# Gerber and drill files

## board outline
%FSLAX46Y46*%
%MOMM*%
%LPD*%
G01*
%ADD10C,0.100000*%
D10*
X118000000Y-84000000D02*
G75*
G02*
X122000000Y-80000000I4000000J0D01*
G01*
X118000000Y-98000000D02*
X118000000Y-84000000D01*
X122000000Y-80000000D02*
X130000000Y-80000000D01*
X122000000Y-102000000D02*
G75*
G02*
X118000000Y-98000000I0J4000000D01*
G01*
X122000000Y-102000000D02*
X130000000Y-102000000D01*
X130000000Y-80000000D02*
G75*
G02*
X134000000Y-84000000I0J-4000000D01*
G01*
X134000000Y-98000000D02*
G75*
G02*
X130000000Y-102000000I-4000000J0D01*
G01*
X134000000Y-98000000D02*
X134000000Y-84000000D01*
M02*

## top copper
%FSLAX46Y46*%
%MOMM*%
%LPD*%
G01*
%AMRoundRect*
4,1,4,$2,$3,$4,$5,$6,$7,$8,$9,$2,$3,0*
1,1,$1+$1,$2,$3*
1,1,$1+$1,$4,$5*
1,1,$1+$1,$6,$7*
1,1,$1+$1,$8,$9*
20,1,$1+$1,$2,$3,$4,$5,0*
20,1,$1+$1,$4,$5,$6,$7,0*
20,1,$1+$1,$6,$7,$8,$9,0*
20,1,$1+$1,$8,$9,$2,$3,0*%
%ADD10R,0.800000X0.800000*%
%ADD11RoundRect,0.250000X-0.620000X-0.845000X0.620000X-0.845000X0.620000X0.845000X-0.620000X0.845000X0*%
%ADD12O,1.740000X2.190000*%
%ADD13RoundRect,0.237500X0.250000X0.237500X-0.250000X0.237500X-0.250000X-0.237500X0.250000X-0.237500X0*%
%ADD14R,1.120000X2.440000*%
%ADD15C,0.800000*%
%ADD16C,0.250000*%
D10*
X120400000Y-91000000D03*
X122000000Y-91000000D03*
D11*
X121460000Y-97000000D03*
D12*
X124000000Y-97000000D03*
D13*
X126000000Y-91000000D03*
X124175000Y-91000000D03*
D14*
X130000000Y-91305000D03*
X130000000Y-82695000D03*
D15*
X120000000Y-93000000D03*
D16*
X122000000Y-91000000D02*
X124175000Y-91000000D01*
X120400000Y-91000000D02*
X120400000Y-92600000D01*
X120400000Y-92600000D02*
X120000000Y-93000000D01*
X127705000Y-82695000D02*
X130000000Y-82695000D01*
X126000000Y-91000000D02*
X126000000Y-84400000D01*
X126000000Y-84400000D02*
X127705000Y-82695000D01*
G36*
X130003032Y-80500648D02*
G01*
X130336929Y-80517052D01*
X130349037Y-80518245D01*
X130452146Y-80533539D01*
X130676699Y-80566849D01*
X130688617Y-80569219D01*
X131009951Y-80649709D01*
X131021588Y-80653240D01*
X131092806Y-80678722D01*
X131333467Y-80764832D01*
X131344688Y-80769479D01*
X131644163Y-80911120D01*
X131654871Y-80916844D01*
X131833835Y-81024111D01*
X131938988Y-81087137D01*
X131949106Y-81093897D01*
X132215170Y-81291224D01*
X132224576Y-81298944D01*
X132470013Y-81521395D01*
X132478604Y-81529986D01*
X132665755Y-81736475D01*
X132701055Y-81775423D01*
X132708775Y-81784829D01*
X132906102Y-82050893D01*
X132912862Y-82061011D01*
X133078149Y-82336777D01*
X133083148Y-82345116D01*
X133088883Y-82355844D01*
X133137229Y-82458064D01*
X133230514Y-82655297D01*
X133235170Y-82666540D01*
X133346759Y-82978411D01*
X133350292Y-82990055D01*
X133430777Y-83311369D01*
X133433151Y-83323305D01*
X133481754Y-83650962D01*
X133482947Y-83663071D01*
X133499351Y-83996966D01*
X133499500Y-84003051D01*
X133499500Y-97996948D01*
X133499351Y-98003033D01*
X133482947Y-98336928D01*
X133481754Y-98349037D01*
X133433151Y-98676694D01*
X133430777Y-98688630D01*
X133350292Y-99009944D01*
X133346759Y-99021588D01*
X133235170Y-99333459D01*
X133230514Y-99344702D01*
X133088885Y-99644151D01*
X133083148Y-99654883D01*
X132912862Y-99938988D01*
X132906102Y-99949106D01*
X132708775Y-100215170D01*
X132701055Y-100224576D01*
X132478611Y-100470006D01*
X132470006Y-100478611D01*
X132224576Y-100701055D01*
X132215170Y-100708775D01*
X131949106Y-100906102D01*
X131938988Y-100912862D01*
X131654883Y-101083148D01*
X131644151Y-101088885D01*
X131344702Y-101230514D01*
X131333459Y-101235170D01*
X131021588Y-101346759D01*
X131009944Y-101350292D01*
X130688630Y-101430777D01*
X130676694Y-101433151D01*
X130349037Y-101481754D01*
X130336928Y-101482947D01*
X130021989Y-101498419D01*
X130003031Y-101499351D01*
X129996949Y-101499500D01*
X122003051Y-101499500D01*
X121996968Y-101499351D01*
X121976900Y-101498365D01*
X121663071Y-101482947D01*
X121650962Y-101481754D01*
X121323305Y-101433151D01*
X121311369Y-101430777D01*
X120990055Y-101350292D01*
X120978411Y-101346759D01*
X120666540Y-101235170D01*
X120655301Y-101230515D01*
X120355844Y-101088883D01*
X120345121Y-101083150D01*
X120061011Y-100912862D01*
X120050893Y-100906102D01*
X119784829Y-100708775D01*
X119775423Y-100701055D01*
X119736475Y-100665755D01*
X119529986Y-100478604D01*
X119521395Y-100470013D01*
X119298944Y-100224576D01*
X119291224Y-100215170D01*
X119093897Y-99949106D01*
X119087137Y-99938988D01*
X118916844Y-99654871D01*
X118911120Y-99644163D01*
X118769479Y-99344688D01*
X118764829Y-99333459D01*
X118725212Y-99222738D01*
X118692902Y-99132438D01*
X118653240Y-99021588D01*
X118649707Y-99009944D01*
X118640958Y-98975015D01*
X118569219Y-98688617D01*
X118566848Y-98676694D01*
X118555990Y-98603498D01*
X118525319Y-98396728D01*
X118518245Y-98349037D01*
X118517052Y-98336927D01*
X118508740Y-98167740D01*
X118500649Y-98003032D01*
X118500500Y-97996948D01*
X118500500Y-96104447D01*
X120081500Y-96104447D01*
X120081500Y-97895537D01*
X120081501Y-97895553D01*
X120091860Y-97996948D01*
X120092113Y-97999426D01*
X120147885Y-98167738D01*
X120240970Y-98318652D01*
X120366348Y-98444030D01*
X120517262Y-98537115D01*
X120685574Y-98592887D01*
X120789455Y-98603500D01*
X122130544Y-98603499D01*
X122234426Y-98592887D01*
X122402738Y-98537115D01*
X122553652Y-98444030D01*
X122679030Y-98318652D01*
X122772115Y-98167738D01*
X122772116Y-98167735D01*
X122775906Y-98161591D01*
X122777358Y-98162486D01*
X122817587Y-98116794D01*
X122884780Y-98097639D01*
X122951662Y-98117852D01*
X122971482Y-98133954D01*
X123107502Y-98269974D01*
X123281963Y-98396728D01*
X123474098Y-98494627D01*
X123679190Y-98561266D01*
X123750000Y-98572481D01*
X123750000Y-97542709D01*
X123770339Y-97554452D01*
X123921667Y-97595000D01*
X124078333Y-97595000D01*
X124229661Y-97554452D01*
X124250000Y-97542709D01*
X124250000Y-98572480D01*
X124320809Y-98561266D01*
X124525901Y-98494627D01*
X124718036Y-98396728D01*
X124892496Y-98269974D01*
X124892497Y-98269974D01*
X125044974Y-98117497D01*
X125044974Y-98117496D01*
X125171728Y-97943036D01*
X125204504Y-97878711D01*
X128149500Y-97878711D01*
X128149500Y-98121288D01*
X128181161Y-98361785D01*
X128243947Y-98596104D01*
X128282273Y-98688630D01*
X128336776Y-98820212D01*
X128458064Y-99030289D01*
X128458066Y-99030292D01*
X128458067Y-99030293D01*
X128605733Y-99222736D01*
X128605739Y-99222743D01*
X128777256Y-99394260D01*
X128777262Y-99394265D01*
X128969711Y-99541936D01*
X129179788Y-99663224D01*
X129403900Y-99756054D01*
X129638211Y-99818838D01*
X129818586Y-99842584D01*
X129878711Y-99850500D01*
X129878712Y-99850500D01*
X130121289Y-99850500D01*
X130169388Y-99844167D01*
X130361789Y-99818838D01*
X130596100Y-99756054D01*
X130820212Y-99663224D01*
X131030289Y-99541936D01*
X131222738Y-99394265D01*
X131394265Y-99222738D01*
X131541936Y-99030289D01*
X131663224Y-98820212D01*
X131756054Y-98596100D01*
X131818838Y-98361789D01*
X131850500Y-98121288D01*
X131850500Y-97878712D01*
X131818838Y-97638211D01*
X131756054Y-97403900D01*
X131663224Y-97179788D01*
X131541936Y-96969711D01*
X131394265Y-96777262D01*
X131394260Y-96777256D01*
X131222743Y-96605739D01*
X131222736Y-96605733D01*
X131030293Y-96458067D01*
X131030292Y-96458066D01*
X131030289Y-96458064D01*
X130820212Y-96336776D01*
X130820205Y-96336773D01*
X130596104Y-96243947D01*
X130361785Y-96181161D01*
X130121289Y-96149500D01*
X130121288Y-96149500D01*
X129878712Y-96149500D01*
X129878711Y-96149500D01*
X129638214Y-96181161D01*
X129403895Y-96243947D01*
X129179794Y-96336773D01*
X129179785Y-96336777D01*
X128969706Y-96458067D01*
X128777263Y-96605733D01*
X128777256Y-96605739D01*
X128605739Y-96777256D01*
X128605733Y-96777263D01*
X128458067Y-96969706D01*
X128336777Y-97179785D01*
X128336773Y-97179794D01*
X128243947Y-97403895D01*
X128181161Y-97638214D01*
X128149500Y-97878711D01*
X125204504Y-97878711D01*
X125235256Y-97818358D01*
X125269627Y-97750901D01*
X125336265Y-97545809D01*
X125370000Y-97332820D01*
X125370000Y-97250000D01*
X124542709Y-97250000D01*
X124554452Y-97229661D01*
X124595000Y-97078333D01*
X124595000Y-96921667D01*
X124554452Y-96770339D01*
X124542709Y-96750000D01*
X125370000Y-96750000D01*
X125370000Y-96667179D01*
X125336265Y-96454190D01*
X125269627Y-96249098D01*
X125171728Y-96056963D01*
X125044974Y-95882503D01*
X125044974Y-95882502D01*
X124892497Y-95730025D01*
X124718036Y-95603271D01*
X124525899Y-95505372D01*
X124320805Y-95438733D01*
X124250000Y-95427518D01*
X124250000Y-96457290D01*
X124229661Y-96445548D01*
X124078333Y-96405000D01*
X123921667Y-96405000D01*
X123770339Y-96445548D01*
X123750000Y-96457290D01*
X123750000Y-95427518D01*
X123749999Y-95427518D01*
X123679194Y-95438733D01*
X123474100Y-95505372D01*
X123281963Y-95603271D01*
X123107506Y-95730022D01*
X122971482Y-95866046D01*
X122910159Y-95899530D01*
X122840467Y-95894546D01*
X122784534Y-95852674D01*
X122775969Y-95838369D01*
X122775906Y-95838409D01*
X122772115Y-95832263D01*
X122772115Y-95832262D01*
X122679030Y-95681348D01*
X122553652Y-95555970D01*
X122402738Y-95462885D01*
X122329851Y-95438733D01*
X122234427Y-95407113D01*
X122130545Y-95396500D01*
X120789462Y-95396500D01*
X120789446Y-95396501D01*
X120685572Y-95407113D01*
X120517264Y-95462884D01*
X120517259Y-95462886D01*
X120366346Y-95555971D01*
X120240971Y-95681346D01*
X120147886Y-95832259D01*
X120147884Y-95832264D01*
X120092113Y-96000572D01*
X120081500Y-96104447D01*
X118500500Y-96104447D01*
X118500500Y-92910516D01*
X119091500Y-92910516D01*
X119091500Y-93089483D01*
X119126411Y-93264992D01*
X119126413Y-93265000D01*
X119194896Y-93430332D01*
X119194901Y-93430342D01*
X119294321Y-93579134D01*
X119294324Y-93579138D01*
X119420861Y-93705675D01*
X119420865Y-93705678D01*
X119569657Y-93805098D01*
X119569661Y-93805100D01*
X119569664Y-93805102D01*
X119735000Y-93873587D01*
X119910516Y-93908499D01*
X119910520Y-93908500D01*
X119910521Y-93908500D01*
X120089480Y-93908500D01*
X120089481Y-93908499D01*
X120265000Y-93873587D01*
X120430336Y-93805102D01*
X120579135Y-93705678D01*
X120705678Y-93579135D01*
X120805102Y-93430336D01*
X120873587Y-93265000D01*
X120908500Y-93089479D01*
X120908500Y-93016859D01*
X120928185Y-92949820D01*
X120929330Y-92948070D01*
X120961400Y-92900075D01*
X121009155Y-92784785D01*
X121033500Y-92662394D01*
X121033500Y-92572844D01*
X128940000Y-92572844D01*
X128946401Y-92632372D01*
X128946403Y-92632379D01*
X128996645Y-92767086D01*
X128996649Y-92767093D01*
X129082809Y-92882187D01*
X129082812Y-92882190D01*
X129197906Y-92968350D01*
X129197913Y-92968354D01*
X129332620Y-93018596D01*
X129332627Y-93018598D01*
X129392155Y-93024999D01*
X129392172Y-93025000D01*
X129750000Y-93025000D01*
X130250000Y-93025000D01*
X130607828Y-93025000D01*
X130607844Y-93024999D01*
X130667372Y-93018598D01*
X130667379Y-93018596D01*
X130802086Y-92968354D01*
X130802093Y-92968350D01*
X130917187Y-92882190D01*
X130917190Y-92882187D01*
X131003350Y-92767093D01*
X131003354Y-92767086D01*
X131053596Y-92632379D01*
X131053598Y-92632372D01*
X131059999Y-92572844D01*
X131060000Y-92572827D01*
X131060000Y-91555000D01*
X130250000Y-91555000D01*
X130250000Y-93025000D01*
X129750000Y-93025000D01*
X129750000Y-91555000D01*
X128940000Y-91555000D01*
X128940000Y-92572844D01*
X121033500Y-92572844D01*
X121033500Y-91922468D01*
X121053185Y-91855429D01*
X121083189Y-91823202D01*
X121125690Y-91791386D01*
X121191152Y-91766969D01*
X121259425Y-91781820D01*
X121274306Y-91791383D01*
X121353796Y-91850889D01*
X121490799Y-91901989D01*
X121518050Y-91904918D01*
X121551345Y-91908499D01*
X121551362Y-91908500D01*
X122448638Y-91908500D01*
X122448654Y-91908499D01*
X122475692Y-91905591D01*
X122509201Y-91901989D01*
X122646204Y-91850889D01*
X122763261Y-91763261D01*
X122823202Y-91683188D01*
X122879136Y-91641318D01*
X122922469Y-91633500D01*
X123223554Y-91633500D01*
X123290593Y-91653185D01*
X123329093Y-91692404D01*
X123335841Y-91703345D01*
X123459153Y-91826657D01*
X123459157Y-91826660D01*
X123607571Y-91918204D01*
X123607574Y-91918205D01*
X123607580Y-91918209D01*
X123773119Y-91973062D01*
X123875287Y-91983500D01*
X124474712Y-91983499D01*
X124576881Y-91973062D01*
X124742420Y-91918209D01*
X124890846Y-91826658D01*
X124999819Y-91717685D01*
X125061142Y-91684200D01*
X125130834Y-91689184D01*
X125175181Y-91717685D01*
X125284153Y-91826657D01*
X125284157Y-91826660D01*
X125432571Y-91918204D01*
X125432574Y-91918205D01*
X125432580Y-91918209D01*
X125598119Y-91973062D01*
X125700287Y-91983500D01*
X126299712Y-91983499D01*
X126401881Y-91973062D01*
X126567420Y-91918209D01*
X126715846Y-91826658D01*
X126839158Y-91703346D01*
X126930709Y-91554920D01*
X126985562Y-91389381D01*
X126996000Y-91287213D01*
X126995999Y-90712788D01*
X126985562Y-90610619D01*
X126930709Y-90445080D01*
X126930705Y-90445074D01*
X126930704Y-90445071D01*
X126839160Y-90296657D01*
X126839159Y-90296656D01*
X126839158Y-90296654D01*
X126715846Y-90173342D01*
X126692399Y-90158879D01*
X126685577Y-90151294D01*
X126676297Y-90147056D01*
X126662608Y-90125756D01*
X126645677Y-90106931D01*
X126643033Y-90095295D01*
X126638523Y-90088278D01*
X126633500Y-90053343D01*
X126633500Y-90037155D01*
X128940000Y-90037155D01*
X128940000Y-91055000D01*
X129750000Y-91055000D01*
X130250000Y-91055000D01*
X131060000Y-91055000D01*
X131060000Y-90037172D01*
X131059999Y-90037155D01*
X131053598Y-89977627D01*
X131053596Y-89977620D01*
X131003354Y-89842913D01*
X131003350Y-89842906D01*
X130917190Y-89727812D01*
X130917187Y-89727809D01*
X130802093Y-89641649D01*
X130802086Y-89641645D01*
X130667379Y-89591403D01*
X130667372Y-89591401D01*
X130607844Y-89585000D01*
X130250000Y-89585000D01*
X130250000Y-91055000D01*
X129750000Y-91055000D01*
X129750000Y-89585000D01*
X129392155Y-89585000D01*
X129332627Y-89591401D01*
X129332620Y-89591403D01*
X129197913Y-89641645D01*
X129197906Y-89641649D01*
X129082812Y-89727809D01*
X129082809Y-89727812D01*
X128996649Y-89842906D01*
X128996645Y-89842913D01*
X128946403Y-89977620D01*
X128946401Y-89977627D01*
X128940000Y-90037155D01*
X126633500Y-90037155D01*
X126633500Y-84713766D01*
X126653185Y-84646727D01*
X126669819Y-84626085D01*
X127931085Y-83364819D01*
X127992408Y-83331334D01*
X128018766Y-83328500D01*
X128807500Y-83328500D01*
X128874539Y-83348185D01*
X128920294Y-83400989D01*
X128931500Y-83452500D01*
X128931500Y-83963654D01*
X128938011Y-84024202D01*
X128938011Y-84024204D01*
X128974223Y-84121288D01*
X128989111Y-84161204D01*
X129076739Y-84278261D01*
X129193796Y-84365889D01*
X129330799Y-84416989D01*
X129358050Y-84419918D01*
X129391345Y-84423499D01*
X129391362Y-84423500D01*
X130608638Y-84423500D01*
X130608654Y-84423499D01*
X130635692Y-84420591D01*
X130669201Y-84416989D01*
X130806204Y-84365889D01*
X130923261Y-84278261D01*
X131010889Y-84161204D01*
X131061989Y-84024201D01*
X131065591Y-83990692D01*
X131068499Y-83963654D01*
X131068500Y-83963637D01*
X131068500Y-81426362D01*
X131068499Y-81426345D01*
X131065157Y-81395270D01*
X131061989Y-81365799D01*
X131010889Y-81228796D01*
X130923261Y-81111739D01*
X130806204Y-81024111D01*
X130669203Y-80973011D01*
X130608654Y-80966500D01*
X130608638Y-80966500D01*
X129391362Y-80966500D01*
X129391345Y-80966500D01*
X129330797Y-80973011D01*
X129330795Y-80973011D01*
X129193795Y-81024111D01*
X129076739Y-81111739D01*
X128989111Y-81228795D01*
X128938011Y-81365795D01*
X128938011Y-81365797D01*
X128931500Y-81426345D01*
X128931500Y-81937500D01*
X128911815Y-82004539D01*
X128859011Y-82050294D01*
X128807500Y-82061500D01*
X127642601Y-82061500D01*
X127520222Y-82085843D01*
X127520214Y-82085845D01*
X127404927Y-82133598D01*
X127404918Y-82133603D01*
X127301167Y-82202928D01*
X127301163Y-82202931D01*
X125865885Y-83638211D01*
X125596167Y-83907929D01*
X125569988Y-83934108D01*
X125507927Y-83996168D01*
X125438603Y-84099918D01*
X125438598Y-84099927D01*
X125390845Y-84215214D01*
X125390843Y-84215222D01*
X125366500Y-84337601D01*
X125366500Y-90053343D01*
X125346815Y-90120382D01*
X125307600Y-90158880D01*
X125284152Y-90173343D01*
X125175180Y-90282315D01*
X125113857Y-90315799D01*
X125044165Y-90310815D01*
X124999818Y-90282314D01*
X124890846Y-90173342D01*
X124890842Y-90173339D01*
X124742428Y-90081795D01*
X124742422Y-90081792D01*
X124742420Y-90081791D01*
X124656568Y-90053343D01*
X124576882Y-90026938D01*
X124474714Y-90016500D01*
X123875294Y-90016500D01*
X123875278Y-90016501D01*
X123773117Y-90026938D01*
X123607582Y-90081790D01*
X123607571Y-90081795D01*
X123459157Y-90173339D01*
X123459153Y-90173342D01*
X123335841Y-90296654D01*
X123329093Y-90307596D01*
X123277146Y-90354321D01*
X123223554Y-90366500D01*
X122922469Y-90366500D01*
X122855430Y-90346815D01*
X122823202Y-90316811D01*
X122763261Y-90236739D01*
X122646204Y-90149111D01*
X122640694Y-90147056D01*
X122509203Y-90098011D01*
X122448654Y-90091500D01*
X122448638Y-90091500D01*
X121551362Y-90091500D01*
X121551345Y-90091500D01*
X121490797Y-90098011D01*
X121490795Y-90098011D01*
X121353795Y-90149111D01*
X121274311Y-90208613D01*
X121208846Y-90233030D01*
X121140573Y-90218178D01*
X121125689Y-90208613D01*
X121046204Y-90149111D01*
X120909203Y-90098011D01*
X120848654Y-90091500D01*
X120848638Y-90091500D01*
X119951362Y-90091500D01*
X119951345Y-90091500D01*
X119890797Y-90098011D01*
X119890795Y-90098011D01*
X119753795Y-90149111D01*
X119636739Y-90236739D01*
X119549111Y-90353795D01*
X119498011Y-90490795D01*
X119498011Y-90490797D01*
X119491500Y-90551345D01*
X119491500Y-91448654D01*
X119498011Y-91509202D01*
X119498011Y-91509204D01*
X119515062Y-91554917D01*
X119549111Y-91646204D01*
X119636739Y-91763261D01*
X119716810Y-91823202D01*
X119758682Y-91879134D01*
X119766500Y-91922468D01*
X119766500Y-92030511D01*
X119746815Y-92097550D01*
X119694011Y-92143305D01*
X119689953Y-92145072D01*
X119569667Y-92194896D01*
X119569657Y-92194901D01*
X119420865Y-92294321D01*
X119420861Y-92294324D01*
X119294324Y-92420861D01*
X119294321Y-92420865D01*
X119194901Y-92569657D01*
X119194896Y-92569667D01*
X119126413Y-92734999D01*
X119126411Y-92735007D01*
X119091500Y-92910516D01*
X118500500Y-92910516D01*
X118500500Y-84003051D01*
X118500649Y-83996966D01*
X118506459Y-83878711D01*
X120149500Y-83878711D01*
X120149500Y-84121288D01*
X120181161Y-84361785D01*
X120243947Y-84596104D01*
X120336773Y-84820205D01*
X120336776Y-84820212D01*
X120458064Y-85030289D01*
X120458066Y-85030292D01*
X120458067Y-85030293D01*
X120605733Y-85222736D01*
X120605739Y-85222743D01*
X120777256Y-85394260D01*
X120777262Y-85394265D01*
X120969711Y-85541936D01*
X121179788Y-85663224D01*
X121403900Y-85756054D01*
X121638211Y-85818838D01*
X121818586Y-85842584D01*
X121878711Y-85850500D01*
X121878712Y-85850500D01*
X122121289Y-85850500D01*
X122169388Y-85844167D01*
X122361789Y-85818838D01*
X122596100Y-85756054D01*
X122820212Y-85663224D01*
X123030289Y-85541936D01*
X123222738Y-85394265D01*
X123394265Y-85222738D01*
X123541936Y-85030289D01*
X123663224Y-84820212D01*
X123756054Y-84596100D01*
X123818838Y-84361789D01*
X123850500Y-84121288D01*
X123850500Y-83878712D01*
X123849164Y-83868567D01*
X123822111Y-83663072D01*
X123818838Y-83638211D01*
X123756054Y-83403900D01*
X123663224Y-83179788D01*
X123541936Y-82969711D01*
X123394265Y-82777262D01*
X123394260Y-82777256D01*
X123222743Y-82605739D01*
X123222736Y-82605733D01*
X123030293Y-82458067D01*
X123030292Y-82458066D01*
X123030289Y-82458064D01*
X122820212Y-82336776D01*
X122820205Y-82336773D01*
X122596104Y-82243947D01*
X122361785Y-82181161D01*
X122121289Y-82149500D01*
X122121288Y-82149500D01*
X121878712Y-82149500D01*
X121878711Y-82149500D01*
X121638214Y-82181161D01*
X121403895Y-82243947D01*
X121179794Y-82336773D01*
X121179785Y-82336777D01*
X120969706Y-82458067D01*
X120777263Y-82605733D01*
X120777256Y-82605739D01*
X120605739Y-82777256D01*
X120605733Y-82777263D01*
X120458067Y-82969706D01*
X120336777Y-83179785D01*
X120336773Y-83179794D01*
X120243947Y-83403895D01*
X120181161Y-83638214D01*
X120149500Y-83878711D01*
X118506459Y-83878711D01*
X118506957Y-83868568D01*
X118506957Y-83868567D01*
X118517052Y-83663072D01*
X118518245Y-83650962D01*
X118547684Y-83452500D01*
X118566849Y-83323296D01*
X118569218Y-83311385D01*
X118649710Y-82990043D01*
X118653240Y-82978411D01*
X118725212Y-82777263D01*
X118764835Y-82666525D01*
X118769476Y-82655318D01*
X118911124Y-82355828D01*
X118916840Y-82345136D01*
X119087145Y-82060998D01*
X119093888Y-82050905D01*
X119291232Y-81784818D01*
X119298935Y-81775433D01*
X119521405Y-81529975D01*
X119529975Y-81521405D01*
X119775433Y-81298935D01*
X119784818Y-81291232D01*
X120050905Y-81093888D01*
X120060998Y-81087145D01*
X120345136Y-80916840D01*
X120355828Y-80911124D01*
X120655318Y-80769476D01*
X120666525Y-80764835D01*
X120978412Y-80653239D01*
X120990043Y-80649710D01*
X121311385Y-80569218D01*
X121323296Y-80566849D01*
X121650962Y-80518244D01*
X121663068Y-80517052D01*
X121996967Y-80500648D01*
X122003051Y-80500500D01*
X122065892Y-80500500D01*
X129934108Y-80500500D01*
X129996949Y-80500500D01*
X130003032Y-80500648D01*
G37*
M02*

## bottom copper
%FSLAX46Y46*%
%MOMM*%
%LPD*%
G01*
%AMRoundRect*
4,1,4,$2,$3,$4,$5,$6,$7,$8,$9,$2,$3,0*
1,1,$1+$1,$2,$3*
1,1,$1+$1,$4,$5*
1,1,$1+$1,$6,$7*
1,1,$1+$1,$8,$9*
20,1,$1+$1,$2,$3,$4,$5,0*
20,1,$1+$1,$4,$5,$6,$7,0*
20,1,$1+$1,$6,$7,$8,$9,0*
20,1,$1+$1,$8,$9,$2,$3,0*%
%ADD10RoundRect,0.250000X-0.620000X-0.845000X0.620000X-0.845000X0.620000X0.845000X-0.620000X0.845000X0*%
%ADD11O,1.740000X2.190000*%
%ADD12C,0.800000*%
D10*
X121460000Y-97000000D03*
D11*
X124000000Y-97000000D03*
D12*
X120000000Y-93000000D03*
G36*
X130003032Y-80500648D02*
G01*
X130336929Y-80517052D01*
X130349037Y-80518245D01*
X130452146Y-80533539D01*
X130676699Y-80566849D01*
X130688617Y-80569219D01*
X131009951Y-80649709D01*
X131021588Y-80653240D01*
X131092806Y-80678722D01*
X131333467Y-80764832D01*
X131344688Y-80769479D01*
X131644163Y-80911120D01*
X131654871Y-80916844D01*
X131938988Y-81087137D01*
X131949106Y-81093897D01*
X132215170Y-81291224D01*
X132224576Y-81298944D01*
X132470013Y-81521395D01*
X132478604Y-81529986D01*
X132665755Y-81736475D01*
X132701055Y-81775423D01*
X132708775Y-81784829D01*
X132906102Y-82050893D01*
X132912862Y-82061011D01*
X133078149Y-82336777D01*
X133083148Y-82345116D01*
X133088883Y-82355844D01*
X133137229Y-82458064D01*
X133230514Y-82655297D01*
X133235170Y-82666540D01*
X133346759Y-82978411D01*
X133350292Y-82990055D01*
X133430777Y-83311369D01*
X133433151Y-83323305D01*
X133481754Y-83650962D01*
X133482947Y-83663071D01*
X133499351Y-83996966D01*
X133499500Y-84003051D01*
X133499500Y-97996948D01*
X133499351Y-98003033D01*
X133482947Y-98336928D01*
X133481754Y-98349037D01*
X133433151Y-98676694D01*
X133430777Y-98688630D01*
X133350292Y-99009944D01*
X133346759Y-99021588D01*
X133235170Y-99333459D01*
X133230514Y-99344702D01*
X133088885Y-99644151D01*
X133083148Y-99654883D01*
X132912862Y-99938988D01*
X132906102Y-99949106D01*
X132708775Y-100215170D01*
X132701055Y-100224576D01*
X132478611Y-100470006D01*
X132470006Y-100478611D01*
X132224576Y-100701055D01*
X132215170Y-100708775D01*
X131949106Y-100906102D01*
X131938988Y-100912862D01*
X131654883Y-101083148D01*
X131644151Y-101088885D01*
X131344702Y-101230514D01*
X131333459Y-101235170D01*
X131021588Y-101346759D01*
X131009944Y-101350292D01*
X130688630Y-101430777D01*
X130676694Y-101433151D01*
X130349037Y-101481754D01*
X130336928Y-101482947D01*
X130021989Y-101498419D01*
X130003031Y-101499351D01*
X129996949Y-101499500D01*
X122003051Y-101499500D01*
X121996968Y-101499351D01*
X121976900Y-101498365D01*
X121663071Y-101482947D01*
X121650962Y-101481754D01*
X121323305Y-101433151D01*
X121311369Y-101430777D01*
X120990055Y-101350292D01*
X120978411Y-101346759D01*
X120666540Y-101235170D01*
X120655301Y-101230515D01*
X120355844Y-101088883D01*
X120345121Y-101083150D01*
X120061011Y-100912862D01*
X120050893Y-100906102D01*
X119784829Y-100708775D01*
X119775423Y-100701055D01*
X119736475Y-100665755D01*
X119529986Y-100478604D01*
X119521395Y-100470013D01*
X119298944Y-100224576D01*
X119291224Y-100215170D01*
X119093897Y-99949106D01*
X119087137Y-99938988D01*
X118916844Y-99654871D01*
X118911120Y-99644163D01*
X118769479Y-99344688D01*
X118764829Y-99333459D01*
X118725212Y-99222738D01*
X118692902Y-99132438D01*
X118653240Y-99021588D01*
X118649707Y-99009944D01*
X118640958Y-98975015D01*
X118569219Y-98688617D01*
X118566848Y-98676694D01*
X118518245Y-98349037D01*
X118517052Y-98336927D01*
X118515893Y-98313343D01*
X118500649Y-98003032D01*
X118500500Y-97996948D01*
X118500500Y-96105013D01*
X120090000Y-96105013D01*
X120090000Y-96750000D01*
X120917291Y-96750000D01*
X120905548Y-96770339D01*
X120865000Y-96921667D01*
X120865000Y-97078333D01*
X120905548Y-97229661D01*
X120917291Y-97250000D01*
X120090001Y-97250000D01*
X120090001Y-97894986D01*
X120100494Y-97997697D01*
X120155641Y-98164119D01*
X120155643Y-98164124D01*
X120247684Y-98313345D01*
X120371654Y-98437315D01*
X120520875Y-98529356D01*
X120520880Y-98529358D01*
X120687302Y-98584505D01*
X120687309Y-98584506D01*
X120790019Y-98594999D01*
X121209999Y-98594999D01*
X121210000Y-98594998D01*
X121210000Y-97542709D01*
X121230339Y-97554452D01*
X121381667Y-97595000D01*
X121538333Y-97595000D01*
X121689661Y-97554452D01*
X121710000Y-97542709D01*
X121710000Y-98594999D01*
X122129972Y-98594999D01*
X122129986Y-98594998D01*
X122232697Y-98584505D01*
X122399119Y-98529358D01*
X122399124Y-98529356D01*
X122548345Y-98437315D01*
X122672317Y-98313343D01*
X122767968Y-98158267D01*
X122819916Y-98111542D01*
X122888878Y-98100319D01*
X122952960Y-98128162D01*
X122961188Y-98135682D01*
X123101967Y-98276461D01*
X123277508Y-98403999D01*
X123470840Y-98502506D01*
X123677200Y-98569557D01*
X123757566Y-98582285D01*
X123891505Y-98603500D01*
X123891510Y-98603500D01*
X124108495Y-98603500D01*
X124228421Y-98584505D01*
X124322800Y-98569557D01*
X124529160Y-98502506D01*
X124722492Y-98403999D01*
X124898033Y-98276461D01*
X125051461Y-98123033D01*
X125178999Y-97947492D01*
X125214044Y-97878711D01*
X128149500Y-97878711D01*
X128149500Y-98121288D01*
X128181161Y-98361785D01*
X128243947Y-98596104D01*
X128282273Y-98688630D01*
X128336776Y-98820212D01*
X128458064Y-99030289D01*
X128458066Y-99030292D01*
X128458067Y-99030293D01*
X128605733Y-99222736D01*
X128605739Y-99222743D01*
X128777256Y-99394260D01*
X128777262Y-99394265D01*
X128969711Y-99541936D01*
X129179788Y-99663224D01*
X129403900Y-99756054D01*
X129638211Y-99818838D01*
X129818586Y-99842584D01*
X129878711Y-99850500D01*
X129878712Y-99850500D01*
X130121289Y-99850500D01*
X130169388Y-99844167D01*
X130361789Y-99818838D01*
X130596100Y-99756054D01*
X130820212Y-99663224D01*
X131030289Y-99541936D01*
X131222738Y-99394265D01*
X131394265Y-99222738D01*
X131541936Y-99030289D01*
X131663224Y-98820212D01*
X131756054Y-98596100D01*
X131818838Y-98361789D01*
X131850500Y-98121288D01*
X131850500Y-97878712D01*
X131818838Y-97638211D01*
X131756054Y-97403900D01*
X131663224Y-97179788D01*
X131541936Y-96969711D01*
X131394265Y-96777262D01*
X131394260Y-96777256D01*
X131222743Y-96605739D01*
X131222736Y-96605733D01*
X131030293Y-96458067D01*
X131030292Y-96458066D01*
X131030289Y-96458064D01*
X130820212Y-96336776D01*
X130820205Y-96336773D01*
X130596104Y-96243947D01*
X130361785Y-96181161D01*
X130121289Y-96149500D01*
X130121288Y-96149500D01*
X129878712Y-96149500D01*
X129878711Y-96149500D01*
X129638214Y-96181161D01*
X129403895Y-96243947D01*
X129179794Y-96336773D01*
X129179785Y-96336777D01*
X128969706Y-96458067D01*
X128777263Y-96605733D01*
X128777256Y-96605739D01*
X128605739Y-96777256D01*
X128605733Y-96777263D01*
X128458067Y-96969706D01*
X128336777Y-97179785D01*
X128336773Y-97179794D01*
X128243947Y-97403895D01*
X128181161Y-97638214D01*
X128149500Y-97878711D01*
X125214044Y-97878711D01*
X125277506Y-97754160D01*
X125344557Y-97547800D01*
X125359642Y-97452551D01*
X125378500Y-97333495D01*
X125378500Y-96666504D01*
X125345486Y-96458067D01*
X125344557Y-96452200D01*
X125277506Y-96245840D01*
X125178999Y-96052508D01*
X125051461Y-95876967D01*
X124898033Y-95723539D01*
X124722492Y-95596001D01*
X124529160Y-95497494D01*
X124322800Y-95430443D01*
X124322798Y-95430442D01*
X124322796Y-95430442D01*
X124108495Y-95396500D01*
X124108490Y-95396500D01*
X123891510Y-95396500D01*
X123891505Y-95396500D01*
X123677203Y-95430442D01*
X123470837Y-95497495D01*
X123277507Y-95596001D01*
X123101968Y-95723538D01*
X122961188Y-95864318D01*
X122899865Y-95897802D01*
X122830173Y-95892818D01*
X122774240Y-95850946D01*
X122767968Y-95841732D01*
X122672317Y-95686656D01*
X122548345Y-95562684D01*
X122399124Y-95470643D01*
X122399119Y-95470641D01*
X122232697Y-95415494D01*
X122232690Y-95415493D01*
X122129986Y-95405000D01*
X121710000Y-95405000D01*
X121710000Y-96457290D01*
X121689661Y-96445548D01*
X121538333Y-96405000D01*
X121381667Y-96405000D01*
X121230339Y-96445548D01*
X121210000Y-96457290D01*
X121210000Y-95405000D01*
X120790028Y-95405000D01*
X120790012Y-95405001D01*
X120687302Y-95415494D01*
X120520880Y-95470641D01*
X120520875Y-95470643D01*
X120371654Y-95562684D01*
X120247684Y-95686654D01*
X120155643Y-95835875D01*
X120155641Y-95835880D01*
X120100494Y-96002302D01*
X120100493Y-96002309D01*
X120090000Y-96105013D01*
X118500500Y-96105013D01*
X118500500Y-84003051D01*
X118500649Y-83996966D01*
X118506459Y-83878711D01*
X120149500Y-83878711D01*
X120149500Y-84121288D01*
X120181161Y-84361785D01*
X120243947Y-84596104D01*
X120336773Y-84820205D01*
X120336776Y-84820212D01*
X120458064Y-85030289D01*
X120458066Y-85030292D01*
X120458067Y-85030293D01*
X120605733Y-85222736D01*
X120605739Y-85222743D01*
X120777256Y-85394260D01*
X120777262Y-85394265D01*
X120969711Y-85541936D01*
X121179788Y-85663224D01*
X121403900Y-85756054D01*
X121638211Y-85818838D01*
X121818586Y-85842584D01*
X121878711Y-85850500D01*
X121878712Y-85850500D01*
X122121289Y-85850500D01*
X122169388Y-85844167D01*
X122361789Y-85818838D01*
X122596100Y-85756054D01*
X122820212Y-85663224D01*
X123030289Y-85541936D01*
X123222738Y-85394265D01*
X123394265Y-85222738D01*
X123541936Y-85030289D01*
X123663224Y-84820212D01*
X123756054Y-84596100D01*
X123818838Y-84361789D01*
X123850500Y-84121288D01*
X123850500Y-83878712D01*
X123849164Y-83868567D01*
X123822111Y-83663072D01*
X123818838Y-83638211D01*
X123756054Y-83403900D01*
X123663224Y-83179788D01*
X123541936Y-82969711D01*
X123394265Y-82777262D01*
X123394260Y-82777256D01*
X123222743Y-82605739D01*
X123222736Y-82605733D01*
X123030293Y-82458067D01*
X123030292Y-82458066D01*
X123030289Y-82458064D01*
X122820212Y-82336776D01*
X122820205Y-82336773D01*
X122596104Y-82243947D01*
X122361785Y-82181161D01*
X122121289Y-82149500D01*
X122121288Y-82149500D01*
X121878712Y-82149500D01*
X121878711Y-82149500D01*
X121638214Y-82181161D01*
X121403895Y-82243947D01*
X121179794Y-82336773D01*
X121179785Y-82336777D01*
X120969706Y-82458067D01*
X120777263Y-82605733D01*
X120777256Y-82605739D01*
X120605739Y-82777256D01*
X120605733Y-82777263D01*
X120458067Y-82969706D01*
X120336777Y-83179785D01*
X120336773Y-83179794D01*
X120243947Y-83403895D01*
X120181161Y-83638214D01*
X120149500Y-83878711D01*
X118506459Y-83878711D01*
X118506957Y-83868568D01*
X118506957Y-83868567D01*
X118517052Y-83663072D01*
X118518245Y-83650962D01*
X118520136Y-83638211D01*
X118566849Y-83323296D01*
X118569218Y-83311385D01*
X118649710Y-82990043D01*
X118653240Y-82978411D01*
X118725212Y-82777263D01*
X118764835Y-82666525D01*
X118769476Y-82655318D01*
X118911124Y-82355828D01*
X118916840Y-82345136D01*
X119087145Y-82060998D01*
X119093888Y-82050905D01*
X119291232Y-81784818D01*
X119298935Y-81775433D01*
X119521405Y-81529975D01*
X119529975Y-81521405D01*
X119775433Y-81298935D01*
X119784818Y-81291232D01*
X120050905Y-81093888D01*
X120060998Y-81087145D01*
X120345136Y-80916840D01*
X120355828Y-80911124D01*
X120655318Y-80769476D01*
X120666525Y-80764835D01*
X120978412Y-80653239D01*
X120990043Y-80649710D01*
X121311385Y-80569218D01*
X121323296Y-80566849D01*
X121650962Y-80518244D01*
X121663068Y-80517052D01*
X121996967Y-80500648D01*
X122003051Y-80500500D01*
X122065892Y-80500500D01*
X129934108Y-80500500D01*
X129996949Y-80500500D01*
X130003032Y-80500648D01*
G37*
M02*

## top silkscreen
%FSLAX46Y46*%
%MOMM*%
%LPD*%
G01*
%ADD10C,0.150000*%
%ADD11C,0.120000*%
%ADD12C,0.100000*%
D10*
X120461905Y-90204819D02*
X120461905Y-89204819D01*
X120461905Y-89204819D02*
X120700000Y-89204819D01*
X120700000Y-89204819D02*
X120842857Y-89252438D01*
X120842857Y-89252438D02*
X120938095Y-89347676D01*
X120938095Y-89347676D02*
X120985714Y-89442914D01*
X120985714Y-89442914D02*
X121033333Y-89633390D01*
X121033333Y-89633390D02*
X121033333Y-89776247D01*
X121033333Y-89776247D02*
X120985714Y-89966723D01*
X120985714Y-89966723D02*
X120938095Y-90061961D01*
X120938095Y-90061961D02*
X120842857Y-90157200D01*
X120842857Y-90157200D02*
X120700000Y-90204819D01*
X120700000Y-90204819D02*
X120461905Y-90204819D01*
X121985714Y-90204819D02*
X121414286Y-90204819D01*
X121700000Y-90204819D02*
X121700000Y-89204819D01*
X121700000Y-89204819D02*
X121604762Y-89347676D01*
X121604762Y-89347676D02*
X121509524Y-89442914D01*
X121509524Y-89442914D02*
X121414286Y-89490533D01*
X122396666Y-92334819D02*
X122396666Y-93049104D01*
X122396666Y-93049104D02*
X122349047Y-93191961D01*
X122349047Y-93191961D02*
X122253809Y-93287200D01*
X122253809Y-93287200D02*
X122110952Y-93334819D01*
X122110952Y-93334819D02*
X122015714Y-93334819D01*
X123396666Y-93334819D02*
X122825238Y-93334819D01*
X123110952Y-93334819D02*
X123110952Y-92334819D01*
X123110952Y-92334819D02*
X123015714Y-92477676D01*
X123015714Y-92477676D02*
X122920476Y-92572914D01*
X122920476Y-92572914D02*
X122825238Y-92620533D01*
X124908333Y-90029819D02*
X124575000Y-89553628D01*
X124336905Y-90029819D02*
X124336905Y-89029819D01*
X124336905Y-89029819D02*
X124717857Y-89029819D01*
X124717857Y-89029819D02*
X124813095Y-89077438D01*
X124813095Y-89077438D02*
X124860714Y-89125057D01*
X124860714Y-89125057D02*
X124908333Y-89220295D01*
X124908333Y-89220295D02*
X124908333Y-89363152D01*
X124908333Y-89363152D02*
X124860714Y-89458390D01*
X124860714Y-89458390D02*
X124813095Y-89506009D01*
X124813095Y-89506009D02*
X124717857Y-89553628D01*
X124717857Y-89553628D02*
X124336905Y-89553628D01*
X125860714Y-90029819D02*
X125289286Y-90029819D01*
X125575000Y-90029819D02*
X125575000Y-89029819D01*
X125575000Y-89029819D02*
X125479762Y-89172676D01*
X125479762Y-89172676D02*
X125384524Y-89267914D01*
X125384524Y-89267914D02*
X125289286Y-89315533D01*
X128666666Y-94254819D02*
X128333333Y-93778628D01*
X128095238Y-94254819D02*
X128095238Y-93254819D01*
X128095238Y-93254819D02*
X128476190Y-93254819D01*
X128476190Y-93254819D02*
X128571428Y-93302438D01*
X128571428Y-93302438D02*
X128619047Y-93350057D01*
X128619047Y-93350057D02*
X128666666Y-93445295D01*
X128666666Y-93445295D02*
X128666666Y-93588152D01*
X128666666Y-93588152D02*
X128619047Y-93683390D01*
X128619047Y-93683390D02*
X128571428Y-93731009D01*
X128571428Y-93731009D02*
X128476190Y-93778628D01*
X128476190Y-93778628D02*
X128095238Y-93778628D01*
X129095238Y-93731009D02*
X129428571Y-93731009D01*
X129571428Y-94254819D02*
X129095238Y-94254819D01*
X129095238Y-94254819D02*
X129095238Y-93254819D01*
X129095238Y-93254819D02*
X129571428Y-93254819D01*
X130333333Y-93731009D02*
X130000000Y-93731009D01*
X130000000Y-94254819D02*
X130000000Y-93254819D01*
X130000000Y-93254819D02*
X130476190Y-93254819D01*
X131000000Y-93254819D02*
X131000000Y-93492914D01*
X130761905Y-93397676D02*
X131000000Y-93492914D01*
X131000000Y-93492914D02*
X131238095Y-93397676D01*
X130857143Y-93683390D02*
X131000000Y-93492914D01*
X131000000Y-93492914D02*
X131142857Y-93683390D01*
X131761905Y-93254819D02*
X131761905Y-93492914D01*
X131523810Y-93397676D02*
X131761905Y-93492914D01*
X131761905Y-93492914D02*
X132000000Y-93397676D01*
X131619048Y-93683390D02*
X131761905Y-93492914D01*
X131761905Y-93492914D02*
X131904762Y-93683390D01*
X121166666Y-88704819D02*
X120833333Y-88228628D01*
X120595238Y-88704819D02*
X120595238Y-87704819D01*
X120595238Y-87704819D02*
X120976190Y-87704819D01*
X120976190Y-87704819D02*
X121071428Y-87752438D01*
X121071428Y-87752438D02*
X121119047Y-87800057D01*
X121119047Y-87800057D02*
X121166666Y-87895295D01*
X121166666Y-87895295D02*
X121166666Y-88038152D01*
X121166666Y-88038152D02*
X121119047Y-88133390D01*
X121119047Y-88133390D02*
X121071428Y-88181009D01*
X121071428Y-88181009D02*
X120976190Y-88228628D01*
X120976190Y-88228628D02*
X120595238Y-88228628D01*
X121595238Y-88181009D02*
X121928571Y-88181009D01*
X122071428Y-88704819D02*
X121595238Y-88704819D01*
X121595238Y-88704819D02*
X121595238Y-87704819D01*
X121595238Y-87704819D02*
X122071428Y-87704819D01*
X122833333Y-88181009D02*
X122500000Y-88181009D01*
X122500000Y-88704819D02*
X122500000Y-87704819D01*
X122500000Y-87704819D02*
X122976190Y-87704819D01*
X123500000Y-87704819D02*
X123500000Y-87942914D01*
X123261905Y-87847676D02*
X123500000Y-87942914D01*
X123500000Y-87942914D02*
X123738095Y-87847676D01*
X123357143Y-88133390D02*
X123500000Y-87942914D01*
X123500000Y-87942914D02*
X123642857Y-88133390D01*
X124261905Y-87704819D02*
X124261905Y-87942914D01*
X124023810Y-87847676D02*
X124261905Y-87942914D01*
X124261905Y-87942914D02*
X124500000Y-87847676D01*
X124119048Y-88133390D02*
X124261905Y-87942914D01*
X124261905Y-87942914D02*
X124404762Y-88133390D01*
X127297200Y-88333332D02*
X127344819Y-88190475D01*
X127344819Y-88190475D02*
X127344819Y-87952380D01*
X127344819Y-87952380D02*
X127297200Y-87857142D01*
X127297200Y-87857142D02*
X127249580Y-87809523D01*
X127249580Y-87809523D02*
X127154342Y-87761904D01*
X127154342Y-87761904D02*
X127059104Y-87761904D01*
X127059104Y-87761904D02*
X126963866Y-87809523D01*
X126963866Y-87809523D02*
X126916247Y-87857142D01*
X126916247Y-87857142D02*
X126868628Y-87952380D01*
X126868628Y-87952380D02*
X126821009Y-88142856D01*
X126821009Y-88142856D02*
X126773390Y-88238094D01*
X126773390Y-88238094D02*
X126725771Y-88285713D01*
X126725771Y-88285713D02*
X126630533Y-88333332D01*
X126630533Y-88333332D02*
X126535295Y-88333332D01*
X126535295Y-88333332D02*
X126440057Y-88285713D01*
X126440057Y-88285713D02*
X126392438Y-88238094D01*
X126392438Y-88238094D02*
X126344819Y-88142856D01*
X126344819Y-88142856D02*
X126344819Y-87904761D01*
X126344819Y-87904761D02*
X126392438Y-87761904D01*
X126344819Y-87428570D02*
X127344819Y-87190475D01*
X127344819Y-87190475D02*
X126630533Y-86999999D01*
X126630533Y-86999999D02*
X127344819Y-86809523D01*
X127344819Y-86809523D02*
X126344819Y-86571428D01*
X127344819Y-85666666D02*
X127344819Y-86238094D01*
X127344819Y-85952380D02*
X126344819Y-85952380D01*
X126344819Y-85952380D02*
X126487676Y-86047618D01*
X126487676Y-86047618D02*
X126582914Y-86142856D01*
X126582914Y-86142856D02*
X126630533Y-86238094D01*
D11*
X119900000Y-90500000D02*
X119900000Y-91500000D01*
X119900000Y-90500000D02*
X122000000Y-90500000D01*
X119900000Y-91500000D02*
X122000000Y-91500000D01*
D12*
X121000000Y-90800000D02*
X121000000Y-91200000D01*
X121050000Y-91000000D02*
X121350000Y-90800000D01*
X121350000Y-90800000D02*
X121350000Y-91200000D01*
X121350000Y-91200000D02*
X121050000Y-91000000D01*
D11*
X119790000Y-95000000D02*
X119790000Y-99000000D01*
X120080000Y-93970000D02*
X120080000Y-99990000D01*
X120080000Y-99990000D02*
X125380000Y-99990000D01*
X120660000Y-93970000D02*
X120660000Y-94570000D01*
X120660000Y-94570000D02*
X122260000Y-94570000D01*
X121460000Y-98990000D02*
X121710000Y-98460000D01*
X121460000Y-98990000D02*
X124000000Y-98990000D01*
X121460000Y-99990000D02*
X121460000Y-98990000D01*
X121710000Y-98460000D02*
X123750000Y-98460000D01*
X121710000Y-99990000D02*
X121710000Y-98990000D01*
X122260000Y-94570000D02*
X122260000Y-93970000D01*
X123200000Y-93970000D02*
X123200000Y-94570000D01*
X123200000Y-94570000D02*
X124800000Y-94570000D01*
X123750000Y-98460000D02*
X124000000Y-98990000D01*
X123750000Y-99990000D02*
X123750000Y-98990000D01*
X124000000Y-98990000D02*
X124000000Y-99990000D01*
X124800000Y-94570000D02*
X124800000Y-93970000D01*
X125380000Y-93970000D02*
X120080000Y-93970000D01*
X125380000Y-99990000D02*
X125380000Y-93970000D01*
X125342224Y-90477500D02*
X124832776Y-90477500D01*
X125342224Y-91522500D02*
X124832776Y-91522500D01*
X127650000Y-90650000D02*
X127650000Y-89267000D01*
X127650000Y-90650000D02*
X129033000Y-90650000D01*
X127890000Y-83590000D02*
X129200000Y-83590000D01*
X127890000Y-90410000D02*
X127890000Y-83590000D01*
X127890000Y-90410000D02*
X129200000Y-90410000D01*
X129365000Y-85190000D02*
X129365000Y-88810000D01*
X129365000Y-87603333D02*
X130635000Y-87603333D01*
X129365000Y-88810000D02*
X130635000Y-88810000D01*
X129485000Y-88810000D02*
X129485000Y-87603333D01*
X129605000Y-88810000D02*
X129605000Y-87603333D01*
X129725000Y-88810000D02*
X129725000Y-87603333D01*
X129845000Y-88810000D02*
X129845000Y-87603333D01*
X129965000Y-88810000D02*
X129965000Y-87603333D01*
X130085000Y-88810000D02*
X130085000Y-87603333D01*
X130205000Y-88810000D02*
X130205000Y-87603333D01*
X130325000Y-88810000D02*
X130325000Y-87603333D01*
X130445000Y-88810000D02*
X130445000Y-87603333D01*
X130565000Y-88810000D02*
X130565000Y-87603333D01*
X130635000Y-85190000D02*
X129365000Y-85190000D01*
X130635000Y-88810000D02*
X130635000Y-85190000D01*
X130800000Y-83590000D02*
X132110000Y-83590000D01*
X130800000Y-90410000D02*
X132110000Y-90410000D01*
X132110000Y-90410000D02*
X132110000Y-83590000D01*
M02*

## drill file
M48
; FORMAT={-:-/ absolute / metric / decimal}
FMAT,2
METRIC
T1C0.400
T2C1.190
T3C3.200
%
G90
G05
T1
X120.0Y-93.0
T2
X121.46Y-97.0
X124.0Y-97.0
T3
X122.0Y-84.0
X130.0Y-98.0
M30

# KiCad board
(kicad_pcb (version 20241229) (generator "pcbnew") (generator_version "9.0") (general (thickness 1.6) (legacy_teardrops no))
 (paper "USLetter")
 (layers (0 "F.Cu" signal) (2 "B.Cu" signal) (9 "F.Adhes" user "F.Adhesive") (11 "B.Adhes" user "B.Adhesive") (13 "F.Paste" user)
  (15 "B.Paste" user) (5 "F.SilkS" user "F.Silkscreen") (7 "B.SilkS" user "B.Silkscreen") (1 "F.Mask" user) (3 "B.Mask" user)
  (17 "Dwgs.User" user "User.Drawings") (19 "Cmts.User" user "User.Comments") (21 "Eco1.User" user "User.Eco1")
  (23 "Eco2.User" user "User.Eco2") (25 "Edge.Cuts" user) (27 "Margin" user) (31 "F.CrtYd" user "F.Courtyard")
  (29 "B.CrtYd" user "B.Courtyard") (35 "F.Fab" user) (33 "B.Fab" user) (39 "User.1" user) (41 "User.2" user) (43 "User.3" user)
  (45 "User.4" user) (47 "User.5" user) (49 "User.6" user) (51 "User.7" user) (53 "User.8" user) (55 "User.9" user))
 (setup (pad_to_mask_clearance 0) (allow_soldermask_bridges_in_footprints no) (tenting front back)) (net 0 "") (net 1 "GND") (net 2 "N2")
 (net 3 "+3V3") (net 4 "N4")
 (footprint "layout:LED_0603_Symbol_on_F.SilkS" (layer "F.Cu") (at 121.2 91)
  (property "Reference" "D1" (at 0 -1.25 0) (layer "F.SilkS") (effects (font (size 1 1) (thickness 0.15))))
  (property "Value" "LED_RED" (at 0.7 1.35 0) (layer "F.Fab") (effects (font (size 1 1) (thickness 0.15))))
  (fp_line (start -1.3 -0.5) (end -1.3 0.5) (stroke (width 0.12) (type solid)) (layer "F.SilkS"))
  (fp_line (start -1.3 -0.5) (end 0.8 -0.5) (stroke (width 0.12) (type solid)) (layer "F.SilkS"))
  (fp_line (start -1.3 0.5) (end 0.8 0.5) (stroke (width 0.12) (type solid)) (layer "F.SilkS"))
  (fp_line (start -0.2 -0.2) (end -0.2 0.2) (stroke (width 0.1) (type solid)) (layer "F.SilkS"))
  (fp_line (start -0.15 0) (end 0.15 -0.2) (stroke (width 0.1) (type solid)) (layer "F.SilkS"))
  (fp_line (start 0.15 -0.2) (end 0.15 0.2) (stroke (width 0.1) (type solid)) (layer "F.SilkS"))
  (fp_line (start 0.15 0.2) (end -0.15 0) (stroke (width 0.1) (type solid)) (layer "F.SilkS"))
  (pad "1" smd rect (at -0.8 0 180) (size 0.8 0.8) (layers "F.Cu" "F.Mask" "F.Paste") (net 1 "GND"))
  (pad "2" smd rect (at 0.8 0 180) (size 0.8 0.8) (layers "F.Cu" "F.Mask" "F.Paste") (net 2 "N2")))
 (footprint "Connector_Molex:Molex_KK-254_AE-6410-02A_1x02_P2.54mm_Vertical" (layer "F.Cu") (at 121.46 97)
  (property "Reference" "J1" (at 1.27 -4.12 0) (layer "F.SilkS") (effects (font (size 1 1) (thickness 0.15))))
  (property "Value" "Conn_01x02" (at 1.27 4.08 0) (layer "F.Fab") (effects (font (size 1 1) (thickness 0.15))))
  (fp_line (start -1.67 -2) (end -1.67 2) (stroke (width 0.12) (type solid)) (layer "F.SilkS"))
  (fp_line (start -1.38 -3.03) (end -1.38 2.99) (stroke (width 0.12) (type solid)) (layer "F.SilkS"))
  (fp_line (start -1.38 2.99) (end 3.92 2.99) (stroke (width 0.12) (type solid)) (layer "F.SilkS"))
  (fp_line (start -0.8 -3.03) (end -0.8 -2.43) (stroke (width 0.12) (type solid)) (layer "F.SilkS"))
  (fp_line (start -0.8 -2.43) (end 0.8 -2.43) (stroke (width 0.12) (type solid)) (layer "F.SilkS"))
  (fp_line (start 0 1.99) (end 0.25 1.46) (stroke (width 0.12) (type solid)) (layer "F.SilkS"))
  (fp_line (start 0 1.99) (end 2.54 1.99) (stroke (width 0.12) (type solid)) (layer "F.SilkS"))
  (fp_line (start 0 2.99) (end 0 1.99) (stroke (width 0.12) (type solid)) (layer "F.SilkS"))
  (fp_line (start 0.25 1.46) (end 2.29 1.46) (stroke (width 0.12) (type solid)) (layer "F.SilkS"))
  (fp_line (start 0.25 2.99) (end 0.25 1.99) (stroke (width 0.12) (type solid)) (layer "F.SilkS"))
  (fp_line (start 0.8 -2.43) (end 0.8 -3.03) (stroke (width 0.12) (type solid)) (layer "F.SilkS"))
  (fp_line (start 1.74 -3.03) (end 1.74 -2.43) (stroke (width 0.12) (type solid)) (layer "F.SilkS"))
  (fp_line (start 1.74 -2.43) (end 3.34 -2.43) (stroke (width 0.12) (type solid)) (layer "F.SilkS"))
  (fp_line (start 2.29 1.46) (end 2.54 1.99) (stroke (width 0.12) (type solid)) (layer "F.SilkS"))
  (fp_line (start 2.29 2.99) (end 2.29 1.99) (stroke (width 0.12) (type solid)) (layer "F.SilkS"))
  (fp_line (start 2.54 1.99) (end 2.54 2.99) (stroke (width 0.12) (type solid)) (layer "F.SilkS"))
  (fp_line (start 3.34 -2.43) (end 3.34 -3.03) (stroke (width 0.12) (type solid)) (layer "F.SilkS"))
  (fp_line (start 3.92 -3.03) (end -1.38 -3.03) (stroke (width 0.12) (type solid)) (layer "F.SilkS"))
  (fp_line (start 3.92 2.99) (end 3.92 -3.03) (stroke (width 0.12) (type solid)) (layer "F.SilkS"))
  (pad "1" thru_hole roundrect (at 0 0) (size 1.74 2.19) (drill 1.19) (layers "*.Cu" "*.Mask") (remove_unused_layers no)
   (roundrect_rratio 0.143678) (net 1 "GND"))
  (pad "2" thru_hole oval (at 2.54 0) (size 1.74 2.19) (drill 1.19) (layers "*.Cu" "*.Mask") (remove_unused_layers no) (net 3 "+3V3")))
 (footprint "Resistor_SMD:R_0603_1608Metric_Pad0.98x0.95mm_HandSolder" (layer "F.Cu") (at 125.0875 91 180)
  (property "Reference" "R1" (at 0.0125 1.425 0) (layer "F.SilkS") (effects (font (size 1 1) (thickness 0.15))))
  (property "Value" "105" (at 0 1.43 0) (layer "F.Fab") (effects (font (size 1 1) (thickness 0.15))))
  (fp_line (start -0.254724 0.5225) (end 0.254724 0.5225) (stroke (width 0.12) (type solid)) (layer "F.SilkS"))
  (fp_line (start -0.254724 -0.5225) (end 0.254724 -0.5225) (stroke (width 0.12) (type solid)) (layer "F.SilkS"))
  (pad "1" smd roundrect (at -0.9125 0 180) (size 0.975 0.95) (layers "F.Cu" "F.Mask" "F.Paste") (roundrect_rratio 0.25) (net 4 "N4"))
  (pad "2" smd roundrect (at 0.9125 0 180) (size 0.975 0.95) (layers "F.Cu" "F.Mask" "F.Paste") (roundrect_rratio 0.25) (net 2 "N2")))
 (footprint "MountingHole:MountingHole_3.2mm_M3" (layer "F.Cu") (at 130 98)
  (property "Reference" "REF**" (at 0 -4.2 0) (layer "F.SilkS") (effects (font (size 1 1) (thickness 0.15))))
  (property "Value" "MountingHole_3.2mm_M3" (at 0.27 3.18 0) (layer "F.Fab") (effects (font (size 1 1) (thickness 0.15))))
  (pad "" np_thru_hole circle (at 0 0) (size 3.2 3.2) (drill 3.2) (layers "*.Cu" "*.Mask")))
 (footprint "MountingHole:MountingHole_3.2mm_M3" (layer "F.Cu") (at 122 84)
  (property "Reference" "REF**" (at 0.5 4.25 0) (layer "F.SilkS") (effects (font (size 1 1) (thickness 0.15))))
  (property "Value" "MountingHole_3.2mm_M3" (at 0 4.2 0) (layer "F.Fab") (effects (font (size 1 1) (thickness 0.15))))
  (pad "" np_thru_hole circle (at 0 0) (size 3.2 3.2) (drill 3.2) (layers "*.Cu" "*.Mask")))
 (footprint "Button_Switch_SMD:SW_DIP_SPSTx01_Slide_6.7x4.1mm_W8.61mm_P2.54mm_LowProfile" (layer "F.Cu") (at 130 87 90)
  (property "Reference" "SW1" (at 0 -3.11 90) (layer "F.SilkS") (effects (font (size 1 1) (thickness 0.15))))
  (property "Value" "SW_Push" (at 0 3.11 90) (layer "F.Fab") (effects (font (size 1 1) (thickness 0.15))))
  (fp_line (start -3.65 -2.35) (end -2.267 -2.35) (stroke (width 0.12) (type solid)) (layer "F.SilkS"))
  (fp_line (start -3.65 -2.35) (end -3.65 -0.967) (stroke (width 0.12) (type solid)) (layer "F.SilkS"))
  (fp_line (start 3.41 -2.11) (end 3.41 -0.8) (stroke (width 0.12) (type solid)) (layer "F.SilkS"))
  (fp_line (start -3.41 -2.11) (end 3.41 -2.11) (stroke (width 0.12) (type solid)) (layer "F.SilkS"))
  (fp_line (start -3.41 -2.11) (end -3.41 -0.8) (stroke (width 0.12) (type solid)) (layer "F.SilkS"))
  (fp_line (start 1.81 -0.635) (end -1.81 -0.635) (stroke (width 0.12) (type solid)) (layer "F.SilkS"))
  (fp_line (start -0.603333 -0.635) (end -0.603333 0.635) (stroke (width 0.12) (type solid)) (layer "F.SilkS"))
  (fp_line (start -1.81 -0.635) (end -1.81 0.635) (stroke (width 0.12) (type solid)) (layer "F.SilkS"))
  (fp_line (start -1.81 -0.515) (end -0.603333 -0.515) (stroke (width 0.12) (type solid)) (layer "F.SilkS"))
  (fp_line (start -1.81 -0.395) (end -0.603333 -0.395) (stroke (width 0.12) (type solid)) (layer "F.SilkS"))
  (fp_line (start -1.81 -0.275) (end -0.603333 -0.275) (stroke (width 0.12) (type solid)) (layer "F.SilkS"))
  (fp_line (start -1.81 -0.155) (end -0.603333 -0.155) (stroke (width 0.12) (type solid)) (layer "F.SilkS"))
  (fp_line (start -1.81 -0.035) (end -0.603333 -0.035) (stroke (width 0.12) (type solid)) (layer "F.SilkS"))
  (fp_line (start -1.81 0.085) (end -0.603333 0.085) (stroke (width 0.12) (type solid)) (layer "F.SilkS"))
  (fp_line (start -1.81 0.205) (end -0.603333 0.205) (stroke (width 0.12) (type solid)) (layer "F.SilkS"))
  (fp_line (start -1.81 0.325) (end -0.603333 0.325) (stroke (width 0.12) (type solid)) (layer "F.SilkS"))
  (fp_line (start -1.81 0.445) (end -0.603333 0.445) (stroke (width 0.12) (type solid)) (layer "F.SilkS"))
  (fp_line (start -1.81 0.565) (end -0.603333 0.565) (stroke (width 0.12) (type solid)) (layer "F.SilkS"))
  (fp_line (start 1.81 0.635) (end 1.81 -0.635) (stroke (width 0.12) (type solid)) (layer "F.SilkS"))
  (fp_line (start -1.81 0.635) (end 1.81 0.635) (stroke (width 0.12) (type solid)) (layer "F.SilkS"))
  (fp_line (start 3.41 0.8) (end 3.41 2.11) (stroke (width 0.12) (type solid)) (layer "F.SilkS"))
  (fp_line (start -3.41 0.8) (end -3.41 2.11) (stroke (width 0.12) (type solid)) (layer "F.SilkS"))
  (fp_line (start -3.41 2.11) (end 3.41 2.11) (stroke (width 0.12) (type solid)) (layer "F.SilkS"))
  (pad "1" smd rect (at -4.305 0 90) (size 2.44 1.12) (layers "F.Cu" "F.Mask" "F.Paste") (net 3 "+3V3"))
  (pad "2" smd rect (at 4.305 0 90) (size 2.44 1.12) (layers "F.Cu" "F.Mask" "F.Paste") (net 4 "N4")))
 (gr_arc (start 118 84) (mid 119.171573 81.171573) (end 122 80) (stroke (width 0.1) (type default)) (layer "Edge.Cuts"))
 (gr_line (start 118 98) (end 118 84) (stroke (width 0.1) (type default)) (layer "Edge.Cuts"))
 (gr_line (start 122 80) (end 130 80) (stroke (width 0.1) (type default)) (layer "Edge.Cuts"))
 (gr_arc (start 122 102) (mid 119.171573 100.828427) (end 118 98) (stroke (width 0.1) (type default)) (layer "Edge.Cuts"))
 (gr_line (start 122 102) (end 130 102) (stroke (width 0.1) (type default)) (layer "Edge.Cuts"))
 (gr_arc (start 130 80) (mid 132.828427 81.171573) (end 134 84) (stroke (width 0.1) (type default)) (layer "Edge.Cuts"))
 (gr_arc (start 134 98) (mid 132.828427 100.828427) (end 130 102) (stroke (width 0.1) (type default)) (layer "Edge.Cuts"))
 (gr_line (start 134 98) (end 134 84) (stroke (width 0.1) (type default)) (layer "Edge.Cuts"))
 (segment (start 122 91) (end 124.175 91) (width 0.25) (layer "F.Cu") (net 2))
 (segment (start 120.4 91) (end 120.4 92.6) (width 0.25) (layer "F.Cu") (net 1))
 (segment (start 120.4 92.6) (end 120 93) (width 0.25) (layer "F.Cu") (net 1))
 (via (at 120 93) (size 0.8) (drill 0.4) (layers "F.Cu" "B.Cu") (free yes) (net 1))
 (segment (start 127.705 82.695) (end 130 82.695) (width 0.25) (layer "F.Cu") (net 4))
 (segment (start 126 91) (end 126 84.4) (width 0.25) (layer "F.Cu") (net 4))
 (segment (start 126 84.4) (end 127.705 82.695) (width 0.25) (layer "F.Cu") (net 4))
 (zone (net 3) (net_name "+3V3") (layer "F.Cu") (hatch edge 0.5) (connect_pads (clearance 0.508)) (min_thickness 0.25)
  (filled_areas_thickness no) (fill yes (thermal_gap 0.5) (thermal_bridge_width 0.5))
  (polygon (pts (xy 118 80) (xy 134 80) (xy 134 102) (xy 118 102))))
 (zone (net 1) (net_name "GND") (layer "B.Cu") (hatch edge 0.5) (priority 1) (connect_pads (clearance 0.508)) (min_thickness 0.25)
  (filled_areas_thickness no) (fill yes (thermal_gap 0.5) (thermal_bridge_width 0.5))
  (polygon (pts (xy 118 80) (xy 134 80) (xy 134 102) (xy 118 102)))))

